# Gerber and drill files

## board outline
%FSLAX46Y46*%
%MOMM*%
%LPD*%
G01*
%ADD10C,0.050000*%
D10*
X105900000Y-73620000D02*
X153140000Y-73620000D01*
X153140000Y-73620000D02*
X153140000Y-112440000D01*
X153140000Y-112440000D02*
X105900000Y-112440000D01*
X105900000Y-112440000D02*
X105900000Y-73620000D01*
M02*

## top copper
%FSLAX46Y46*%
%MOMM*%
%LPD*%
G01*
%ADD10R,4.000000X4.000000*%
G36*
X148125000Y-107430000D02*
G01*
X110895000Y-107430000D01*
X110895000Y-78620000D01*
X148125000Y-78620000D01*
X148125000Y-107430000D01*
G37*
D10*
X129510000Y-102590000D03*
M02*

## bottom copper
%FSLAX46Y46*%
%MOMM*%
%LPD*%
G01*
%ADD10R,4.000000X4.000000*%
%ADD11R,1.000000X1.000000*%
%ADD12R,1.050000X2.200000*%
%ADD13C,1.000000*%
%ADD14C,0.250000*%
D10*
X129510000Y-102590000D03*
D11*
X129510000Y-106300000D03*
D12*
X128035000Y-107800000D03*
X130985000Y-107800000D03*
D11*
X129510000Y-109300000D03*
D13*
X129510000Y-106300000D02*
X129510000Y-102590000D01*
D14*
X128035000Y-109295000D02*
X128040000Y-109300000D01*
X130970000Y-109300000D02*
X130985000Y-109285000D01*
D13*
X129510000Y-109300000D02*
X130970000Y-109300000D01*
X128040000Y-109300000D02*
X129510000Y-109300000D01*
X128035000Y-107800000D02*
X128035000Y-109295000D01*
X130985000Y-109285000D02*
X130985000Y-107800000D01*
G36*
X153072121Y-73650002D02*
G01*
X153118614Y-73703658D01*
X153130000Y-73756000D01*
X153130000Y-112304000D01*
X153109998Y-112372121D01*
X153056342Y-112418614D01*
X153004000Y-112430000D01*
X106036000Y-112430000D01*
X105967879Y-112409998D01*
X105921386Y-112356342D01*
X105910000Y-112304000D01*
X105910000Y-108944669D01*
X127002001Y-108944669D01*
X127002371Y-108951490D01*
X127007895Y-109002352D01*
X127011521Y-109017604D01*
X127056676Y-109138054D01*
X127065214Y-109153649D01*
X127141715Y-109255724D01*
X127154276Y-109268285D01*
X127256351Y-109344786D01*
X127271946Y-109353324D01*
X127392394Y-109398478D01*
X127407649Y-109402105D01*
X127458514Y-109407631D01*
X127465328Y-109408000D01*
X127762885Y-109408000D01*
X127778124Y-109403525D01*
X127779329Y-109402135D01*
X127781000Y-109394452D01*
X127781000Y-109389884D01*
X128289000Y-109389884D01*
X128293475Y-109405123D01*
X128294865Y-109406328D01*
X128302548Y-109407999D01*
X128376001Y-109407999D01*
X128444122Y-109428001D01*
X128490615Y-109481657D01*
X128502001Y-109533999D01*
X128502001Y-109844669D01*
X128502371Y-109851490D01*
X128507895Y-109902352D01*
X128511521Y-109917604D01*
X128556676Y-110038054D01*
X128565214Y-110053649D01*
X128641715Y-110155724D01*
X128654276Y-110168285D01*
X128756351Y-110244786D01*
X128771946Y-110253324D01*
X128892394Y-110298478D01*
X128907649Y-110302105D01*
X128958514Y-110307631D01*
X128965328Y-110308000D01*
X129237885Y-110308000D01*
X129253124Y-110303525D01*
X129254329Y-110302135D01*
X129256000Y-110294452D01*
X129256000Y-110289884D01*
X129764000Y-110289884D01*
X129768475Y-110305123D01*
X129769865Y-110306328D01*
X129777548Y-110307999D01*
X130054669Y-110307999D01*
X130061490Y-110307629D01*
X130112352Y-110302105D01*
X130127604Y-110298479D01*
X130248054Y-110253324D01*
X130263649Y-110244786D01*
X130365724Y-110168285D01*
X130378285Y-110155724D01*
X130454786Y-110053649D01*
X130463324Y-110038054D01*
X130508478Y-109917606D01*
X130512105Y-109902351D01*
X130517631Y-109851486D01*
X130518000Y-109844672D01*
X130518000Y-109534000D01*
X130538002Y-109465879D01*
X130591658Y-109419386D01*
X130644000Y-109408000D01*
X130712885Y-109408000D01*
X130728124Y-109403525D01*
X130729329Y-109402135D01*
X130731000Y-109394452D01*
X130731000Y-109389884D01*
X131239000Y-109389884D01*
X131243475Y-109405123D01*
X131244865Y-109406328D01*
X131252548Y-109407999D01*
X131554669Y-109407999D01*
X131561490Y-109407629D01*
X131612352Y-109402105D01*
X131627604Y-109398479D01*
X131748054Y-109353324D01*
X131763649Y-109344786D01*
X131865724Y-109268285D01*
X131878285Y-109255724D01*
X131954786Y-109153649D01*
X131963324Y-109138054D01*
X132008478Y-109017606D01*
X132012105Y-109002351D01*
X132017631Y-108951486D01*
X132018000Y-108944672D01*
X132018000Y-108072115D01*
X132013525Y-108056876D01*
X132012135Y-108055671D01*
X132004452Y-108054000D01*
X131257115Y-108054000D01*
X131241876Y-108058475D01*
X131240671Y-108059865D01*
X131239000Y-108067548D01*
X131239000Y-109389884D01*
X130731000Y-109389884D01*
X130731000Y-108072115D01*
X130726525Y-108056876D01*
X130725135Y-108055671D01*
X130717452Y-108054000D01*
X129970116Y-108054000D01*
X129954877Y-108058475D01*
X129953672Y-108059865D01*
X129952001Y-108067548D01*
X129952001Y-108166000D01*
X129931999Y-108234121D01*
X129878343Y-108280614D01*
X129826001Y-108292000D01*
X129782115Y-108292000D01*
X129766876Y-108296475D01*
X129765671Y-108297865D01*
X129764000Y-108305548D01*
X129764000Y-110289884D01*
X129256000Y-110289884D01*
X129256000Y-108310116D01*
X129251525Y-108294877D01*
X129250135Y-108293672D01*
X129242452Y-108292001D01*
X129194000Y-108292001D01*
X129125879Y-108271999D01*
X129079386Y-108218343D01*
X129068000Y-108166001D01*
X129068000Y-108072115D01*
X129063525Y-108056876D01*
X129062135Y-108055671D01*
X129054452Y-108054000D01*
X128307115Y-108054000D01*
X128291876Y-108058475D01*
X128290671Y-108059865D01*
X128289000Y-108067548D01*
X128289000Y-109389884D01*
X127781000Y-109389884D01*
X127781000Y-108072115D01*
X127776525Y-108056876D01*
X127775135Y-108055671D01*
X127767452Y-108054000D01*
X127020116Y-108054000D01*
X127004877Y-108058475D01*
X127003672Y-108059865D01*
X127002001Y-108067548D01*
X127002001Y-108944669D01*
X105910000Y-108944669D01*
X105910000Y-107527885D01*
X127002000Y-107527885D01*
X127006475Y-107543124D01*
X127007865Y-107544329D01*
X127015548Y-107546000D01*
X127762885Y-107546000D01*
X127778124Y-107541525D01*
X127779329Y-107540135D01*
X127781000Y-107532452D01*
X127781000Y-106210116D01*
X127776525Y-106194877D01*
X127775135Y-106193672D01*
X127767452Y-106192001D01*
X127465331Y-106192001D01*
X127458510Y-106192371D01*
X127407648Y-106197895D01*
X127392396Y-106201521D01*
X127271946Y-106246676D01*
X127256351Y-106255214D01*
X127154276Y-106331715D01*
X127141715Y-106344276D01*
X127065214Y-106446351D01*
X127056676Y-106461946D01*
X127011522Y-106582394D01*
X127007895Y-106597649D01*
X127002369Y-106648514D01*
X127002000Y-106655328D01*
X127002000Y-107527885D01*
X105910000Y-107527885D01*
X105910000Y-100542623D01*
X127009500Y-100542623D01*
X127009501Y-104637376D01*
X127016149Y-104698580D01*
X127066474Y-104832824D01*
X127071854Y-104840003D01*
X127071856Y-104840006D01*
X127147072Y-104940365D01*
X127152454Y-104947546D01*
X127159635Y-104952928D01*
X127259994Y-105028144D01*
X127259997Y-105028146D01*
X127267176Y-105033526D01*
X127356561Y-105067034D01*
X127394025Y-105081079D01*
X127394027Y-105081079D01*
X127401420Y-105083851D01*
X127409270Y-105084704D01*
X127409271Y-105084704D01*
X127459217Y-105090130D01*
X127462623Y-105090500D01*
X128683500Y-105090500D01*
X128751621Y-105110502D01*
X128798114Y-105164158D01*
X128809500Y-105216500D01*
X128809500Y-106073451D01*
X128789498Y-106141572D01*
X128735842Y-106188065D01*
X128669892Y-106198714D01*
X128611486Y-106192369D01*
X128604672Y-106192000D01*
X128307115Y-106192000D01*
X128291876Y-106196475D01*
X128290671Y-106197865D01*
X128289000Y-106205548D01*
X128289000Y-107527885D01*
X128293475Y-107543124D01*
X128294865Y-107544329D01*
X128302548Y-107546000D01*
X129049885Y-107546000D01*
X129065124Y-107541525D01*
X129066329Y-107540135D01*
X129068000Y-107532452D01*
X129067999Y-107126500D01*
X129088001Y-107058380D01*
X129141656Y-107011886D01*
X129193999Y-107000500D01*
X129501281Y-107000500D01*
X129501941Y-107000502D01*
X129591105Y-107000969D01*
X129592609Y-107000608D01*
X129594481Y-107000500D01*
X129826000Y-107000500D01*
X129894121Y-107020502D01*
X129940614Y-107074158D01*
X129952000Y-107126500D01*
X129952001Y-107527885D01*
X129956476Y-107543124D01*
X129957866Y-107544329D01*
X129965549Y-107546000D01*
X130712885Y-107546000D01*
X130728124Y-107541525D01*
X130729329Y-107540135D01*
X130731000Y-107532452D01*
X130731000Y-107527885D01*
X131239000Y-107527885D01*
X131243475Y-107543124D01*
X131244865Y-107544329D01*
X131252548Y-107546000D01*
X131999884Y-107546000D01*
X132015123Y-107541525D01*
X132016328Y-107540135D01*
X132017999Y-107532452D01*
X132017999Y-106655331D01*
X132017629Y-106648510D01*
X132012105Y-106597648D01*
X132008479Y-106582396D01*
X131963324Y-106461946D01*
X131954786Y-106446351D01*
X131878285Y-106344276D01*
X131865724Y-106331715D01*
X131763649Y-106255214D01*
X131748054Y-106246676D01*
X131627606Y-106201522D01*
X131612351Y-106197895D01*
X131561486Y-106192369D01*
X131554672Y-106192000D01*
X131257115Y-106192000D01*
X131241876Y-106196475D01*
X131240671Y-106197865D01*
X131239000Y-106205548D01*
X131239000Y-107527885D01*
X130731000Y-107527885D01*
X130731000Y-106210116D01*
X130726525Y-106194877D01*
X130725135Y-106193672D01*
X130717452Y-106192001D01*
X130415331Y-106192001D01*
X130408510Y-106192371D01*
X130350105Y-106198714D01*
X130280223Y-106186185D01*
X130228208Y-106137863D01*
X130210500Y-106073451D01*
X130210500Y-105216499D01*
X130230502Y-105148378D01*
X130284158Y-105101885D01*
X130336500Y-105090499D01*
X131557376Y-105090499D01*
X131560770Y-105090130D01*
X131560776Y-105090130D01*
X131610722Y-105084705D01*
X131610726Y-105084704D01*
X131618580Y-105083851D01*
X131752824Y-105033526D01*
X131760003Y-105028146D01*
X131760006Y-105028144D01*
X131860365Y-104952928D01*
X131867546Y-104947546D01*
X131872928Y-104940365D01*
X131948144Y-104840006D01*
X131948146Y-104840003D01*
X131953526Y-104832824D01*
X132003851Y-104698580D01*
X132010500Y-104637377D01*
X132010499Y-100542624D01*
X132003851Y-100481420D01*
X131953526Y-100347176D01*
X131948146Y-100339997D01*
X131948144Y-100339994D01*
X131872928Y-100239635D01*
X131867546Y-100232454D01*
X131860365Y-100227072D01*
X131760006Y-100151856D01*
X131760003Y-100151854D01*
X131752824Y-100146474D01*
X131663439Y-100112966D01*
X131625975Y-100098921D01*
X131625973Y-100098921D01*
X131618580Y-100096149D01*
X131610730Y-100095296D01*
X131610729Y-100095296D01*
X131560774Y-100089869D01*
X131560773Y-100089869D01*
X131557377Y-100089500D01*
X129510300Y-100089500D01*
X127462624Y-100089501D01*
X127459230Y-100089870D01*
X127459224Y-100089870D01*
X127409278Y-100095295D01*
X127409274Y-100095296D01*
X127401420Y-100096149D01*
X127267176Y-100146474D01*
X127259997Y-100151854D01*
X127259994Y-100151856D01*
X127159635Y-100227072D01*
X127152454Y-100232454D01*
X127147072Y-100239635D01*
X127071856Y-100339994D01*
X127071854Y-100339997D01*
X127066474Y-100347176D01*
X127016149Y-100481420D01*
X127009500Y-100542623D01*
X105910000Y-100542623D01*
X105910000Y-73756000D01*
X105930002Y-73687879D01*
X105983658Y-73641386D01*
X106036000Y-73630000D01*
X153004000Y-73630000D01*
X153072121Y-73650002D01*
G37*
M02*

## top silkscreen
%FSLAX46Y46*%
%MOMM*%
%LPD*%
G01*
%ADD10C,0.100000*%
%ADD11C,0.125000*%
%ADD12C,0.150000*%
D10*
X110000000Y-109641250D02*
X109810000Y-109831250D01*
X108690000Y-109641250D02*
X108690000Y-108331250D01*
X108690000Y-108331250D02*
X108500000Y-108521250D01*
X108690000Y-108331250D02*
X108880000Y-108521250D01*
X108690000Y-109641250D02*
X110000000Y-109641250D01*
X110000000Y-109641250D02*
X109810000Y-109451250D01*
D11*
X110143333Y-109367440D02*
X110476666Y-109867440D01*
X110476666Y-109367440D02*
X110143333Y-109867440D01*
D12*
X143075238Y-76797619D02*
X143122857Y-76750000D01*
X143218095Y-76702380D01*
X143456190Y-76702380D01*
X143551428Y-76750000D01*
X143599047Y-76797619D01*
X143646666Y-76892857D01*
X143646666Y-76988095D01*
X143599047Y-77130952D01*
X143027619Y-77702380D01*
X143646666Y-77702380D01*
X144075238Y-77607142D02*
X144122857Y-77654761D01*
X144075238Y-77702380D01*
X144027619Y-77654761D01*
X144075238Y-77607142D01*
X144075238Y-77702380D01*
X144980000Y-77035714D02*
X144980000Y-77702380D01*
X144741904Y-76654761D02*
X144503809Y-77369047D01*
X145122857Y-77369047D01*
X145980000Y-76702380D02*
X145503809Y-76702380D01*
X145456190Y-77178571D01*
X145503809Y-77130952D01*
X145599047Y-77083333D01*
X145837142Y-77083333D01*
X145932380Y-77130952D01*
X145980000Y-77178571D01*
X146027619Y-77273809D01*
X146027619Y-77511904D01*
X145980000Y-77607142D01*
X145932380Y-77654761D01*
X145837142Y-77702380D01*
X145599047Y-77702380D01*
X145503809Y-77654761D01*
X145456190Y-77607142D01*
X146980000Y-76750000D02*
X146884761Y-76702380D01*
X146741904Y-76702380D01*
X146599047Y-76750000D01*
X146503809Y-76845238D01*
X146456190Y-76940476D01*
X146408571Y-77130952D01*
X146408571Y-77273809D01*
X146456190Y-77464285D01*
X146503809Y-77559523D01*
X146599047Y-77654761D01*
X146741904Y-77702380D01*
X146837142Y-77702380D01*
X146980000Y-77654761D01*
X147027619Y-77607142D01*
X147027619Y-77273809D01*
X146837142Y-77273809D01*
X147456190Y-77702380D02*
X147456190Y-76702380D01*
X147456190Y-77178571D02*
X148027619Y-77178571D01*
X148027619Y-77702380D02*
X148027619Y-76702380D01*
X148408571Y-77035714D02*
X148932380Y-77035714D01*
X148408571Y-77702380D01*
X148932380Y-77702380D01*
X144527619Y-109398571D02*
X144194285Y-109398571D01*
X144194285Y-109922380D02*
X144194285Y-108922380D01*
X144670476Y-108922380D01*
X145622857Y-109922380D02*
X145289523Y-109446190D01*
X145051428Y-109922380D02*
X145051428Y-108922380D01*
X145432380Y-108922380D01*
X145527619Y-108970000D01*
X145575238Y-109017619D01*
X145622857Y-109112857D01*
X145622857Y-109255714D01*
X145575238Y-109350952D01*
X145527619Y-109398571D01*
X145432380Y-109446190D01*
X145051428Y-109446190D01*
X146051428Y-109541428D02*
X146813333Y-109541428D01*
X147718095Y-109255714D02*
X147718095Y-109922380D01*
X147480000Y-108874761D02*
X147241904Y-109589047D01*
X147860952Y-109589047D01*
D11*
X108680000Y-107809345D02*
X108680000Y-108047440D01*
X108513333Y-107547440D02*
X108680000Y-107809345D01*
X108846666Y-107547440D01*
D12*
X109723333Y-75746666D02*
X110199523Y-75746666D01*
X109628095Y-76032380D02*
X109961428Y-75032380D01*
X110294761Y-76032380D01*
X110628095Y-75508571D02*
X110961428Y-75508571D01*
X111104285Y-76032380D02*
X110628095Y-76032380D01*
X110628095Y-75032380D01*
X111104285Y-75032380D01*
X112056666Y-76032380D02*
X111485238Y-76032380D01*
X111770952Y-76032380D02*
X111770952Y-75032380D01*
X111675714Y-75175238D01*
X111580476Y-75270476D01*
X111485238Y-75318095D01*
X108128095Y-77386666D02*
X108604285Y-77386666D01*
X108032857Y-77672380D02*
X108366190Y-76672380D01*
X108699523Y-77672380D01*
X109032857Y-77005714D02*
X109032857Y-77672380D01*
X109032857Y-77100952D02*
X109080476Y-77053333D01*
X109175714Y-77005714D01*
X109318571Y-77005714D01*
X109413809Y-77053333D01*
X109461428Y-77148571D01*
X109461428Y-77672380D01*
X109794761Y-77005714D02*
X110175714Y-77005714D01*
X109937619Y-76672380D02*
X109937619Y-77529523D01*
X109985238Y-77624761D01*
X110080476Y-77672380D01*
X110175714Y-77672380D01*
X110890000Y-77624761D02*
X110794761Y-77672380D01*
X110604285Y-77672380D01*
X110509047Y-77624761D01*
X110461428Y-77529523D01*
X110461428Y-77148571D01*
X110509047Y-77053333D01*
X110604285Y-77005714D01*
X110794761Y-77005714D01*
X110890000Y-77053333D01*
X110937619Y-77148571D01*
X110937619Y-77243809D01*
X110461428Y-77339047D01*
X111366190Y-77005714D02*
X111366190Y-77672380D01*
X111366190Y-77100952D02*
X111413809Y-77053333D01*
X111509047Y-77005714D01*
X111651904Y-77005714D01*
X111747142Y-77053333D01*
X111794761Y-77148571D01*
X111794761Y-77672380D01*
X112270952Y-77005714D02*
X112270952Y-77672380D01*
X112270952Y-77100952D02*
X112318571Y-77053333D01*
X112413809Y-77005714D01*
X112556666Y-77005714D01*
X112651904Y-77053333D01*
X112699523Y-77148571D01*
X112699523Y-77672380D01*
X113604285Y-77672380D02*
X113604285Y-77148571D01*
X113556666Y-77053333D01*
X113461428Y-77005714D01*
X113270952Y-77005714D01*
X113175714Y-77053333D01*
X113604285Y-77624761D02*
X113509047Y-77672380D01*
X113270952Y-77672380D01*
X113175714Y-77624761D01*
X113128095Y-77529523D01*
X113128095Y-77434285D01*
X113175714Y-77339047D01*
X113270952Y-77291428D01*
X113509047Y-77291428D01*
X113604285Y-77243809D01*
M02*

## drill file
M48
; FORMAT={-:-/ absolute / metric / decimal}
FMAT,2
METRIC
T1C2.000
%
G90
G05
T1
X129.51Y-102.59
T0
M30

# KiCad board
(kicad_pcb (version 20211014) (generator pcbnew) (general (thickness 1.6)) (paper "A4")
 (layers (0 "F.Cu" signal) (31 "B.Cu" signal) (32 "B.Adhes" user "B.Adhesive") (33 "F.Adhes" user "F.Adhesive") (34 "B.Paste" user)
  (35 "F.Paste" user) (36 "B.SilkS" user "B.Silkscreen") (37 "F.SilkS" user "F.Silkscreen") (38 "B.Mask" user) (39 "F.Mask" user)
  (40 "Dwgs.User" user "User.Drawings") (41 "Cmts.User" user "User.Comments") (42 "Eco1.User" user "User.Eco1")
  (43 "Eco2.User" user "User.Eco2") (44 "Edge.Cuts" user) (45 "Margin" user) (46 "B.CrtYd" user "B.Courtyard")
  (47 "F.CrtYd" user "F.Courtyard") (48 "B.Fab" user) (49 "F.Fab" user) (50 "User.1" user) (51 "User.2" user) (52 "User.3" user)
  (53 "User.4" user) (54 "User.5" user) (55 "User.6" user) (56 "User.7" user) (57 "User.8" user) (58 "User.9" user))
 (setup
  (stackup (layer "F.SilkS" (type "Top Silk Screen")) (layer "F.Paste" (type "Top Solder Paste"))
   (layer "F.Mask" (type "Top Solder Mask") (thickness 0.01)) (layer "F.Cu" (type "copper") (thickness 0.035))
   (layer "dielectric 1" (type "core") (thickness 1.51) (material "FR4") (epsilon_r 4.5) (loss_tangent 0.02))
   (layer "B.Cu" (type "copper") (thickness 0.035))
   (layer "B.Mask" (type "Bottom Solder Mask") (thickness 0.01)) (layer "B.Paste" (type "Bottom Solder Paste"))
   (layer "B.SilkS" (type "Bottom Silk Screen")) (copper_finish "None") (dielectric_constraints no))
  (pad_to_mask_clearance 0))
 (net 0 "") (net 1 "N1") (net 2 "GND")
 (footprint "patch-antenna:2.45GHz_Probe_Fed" (layer "F.Cu") (at 110.895 78.62)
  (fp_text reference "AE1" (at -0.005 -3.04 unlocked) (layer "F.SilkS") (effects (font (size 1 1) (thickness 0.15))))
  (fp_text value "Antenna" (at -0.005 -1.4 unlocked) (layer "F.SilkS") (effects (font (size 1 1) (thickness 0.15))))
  (fp_rect (start 37.23 28.81) (end 0 0) (layer "F.Cu") (width 0) (fill solid))
  (pad "1" thru_hole rect (at 18.615 23.97 180) (size 4 4) (drill 2) (layers *.Cu *.Mask) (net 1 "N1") (clearance 0.5)))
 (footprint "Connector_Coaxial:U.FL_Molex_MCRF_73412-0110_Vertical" (layer "B.Cu") (at 129.51 107.8)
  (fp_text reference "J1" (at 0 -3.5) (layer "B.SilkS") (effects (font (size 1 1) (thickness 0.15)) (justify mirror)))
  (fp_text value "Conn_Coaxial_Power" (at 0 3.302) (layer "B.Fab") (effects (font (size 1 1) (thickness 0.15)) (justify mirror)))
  (pad "1" smd rect (at 0 -1.5) (size 1 1) (layers "B.Cu" "B.Paste" "B.Mask") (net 1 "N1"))
  (pad "2" smd rect (at -1.475 0) (size 1.05 2.2) (layers "B.Cu" "B.Paste" "B.Mask") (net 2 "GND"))
  (pad "2" smd rect (at 1.475 0) (size 1.05 2.2) (layers "B.Cu" "B.Paste" "B.Mask") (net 2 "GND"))
  (pad "2" smd rect (at 0 1.5) (size 1 1) (layers "B.Cu" "B.Paste" "B.Mask") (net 2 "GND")))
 (gr_line (start 110 109.64125) (end 109.81 109.83125) (layer "F.SilkS") (width 0.1))
 (gr_line (start 108.69 109.64125) (end 108.69 108.33125) (layer "F.SilkS") (width 0.1))
 (gr_line (start 108.69 108.33125) (end 108.5 108.52125) (layer "F.SilkS") (width 0.1))
 (gr_line (start 108.69 108.33125) (end 108.88 108.52125) (layer "F.SilkS") (width 0.1))
 (gr_line (start 108.69 109.64125) (end 110 109.64125) (layer "F.SilkS") (width 0.1))
 (gr_line (start 110 109.64125) (end 109.81 109.45125) (layer "F.SilkS") (width 0.1))
 (gr_rect (start 105.9 73.62) (end 153.14 112.44) (layer "Edge.Cuts") (width 0.05) (fill none))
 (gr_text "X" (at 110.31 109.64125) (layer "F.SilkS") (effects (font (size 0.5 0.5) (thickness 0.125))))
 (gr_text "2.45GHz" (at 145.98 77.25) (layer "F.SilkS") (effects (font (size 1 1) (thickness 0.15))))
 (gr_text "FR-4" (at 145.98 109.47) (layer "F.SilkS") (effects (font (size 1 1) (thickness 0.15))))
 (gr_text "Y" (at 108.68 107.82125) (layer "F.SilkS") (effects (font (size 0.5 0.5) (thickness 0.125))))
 (segment (start 129.51 106.3) (end 129.51 102.59) (width 1) (layer "B.Cu") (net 1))
 (segment (start 128.035 109.295) (end 128.04 109.3) (width 0.25) (layer "B.Cu") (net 2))
 (segment (start 130.97 109.3) (end 130.985 109.285) (width 0.25) (layer "B.Cu") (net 2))
 (segment (start 129.51 109.3) (end 130.97 109.3) (width 1) (layer "B.Cu") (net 2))
 (segment (start 128.04 109.3) (end 129.51 109.3) (width 1) (layer "B.Cu") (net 2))
 (segment (start 128.035 107.8) (end 128.035 109.295) (width 1) (layer "B.Cu") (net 2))
 (segment (start 130.985 109.285) (end 130.985 107.8) (width 1) (layer "B.Cu") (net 2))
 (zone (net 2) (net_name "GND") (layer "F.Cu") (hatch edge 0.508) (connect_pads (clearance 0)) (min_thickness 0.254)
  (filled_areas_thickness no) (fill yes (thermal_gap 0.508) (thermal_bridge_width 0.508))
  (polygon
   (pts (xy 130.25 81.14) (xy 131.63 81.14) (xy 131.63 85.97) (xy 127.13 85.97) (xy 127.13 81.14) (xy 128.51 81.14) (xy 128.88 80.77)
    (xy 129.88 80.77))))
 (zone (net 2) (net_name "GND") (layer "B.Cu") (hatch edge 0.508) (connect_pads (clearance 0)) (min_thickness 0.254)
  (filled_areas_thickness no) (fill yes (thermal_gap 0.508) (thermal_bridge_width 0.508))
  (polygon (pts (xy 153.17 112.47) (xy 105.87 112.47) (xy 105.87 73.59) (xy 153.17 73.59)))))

